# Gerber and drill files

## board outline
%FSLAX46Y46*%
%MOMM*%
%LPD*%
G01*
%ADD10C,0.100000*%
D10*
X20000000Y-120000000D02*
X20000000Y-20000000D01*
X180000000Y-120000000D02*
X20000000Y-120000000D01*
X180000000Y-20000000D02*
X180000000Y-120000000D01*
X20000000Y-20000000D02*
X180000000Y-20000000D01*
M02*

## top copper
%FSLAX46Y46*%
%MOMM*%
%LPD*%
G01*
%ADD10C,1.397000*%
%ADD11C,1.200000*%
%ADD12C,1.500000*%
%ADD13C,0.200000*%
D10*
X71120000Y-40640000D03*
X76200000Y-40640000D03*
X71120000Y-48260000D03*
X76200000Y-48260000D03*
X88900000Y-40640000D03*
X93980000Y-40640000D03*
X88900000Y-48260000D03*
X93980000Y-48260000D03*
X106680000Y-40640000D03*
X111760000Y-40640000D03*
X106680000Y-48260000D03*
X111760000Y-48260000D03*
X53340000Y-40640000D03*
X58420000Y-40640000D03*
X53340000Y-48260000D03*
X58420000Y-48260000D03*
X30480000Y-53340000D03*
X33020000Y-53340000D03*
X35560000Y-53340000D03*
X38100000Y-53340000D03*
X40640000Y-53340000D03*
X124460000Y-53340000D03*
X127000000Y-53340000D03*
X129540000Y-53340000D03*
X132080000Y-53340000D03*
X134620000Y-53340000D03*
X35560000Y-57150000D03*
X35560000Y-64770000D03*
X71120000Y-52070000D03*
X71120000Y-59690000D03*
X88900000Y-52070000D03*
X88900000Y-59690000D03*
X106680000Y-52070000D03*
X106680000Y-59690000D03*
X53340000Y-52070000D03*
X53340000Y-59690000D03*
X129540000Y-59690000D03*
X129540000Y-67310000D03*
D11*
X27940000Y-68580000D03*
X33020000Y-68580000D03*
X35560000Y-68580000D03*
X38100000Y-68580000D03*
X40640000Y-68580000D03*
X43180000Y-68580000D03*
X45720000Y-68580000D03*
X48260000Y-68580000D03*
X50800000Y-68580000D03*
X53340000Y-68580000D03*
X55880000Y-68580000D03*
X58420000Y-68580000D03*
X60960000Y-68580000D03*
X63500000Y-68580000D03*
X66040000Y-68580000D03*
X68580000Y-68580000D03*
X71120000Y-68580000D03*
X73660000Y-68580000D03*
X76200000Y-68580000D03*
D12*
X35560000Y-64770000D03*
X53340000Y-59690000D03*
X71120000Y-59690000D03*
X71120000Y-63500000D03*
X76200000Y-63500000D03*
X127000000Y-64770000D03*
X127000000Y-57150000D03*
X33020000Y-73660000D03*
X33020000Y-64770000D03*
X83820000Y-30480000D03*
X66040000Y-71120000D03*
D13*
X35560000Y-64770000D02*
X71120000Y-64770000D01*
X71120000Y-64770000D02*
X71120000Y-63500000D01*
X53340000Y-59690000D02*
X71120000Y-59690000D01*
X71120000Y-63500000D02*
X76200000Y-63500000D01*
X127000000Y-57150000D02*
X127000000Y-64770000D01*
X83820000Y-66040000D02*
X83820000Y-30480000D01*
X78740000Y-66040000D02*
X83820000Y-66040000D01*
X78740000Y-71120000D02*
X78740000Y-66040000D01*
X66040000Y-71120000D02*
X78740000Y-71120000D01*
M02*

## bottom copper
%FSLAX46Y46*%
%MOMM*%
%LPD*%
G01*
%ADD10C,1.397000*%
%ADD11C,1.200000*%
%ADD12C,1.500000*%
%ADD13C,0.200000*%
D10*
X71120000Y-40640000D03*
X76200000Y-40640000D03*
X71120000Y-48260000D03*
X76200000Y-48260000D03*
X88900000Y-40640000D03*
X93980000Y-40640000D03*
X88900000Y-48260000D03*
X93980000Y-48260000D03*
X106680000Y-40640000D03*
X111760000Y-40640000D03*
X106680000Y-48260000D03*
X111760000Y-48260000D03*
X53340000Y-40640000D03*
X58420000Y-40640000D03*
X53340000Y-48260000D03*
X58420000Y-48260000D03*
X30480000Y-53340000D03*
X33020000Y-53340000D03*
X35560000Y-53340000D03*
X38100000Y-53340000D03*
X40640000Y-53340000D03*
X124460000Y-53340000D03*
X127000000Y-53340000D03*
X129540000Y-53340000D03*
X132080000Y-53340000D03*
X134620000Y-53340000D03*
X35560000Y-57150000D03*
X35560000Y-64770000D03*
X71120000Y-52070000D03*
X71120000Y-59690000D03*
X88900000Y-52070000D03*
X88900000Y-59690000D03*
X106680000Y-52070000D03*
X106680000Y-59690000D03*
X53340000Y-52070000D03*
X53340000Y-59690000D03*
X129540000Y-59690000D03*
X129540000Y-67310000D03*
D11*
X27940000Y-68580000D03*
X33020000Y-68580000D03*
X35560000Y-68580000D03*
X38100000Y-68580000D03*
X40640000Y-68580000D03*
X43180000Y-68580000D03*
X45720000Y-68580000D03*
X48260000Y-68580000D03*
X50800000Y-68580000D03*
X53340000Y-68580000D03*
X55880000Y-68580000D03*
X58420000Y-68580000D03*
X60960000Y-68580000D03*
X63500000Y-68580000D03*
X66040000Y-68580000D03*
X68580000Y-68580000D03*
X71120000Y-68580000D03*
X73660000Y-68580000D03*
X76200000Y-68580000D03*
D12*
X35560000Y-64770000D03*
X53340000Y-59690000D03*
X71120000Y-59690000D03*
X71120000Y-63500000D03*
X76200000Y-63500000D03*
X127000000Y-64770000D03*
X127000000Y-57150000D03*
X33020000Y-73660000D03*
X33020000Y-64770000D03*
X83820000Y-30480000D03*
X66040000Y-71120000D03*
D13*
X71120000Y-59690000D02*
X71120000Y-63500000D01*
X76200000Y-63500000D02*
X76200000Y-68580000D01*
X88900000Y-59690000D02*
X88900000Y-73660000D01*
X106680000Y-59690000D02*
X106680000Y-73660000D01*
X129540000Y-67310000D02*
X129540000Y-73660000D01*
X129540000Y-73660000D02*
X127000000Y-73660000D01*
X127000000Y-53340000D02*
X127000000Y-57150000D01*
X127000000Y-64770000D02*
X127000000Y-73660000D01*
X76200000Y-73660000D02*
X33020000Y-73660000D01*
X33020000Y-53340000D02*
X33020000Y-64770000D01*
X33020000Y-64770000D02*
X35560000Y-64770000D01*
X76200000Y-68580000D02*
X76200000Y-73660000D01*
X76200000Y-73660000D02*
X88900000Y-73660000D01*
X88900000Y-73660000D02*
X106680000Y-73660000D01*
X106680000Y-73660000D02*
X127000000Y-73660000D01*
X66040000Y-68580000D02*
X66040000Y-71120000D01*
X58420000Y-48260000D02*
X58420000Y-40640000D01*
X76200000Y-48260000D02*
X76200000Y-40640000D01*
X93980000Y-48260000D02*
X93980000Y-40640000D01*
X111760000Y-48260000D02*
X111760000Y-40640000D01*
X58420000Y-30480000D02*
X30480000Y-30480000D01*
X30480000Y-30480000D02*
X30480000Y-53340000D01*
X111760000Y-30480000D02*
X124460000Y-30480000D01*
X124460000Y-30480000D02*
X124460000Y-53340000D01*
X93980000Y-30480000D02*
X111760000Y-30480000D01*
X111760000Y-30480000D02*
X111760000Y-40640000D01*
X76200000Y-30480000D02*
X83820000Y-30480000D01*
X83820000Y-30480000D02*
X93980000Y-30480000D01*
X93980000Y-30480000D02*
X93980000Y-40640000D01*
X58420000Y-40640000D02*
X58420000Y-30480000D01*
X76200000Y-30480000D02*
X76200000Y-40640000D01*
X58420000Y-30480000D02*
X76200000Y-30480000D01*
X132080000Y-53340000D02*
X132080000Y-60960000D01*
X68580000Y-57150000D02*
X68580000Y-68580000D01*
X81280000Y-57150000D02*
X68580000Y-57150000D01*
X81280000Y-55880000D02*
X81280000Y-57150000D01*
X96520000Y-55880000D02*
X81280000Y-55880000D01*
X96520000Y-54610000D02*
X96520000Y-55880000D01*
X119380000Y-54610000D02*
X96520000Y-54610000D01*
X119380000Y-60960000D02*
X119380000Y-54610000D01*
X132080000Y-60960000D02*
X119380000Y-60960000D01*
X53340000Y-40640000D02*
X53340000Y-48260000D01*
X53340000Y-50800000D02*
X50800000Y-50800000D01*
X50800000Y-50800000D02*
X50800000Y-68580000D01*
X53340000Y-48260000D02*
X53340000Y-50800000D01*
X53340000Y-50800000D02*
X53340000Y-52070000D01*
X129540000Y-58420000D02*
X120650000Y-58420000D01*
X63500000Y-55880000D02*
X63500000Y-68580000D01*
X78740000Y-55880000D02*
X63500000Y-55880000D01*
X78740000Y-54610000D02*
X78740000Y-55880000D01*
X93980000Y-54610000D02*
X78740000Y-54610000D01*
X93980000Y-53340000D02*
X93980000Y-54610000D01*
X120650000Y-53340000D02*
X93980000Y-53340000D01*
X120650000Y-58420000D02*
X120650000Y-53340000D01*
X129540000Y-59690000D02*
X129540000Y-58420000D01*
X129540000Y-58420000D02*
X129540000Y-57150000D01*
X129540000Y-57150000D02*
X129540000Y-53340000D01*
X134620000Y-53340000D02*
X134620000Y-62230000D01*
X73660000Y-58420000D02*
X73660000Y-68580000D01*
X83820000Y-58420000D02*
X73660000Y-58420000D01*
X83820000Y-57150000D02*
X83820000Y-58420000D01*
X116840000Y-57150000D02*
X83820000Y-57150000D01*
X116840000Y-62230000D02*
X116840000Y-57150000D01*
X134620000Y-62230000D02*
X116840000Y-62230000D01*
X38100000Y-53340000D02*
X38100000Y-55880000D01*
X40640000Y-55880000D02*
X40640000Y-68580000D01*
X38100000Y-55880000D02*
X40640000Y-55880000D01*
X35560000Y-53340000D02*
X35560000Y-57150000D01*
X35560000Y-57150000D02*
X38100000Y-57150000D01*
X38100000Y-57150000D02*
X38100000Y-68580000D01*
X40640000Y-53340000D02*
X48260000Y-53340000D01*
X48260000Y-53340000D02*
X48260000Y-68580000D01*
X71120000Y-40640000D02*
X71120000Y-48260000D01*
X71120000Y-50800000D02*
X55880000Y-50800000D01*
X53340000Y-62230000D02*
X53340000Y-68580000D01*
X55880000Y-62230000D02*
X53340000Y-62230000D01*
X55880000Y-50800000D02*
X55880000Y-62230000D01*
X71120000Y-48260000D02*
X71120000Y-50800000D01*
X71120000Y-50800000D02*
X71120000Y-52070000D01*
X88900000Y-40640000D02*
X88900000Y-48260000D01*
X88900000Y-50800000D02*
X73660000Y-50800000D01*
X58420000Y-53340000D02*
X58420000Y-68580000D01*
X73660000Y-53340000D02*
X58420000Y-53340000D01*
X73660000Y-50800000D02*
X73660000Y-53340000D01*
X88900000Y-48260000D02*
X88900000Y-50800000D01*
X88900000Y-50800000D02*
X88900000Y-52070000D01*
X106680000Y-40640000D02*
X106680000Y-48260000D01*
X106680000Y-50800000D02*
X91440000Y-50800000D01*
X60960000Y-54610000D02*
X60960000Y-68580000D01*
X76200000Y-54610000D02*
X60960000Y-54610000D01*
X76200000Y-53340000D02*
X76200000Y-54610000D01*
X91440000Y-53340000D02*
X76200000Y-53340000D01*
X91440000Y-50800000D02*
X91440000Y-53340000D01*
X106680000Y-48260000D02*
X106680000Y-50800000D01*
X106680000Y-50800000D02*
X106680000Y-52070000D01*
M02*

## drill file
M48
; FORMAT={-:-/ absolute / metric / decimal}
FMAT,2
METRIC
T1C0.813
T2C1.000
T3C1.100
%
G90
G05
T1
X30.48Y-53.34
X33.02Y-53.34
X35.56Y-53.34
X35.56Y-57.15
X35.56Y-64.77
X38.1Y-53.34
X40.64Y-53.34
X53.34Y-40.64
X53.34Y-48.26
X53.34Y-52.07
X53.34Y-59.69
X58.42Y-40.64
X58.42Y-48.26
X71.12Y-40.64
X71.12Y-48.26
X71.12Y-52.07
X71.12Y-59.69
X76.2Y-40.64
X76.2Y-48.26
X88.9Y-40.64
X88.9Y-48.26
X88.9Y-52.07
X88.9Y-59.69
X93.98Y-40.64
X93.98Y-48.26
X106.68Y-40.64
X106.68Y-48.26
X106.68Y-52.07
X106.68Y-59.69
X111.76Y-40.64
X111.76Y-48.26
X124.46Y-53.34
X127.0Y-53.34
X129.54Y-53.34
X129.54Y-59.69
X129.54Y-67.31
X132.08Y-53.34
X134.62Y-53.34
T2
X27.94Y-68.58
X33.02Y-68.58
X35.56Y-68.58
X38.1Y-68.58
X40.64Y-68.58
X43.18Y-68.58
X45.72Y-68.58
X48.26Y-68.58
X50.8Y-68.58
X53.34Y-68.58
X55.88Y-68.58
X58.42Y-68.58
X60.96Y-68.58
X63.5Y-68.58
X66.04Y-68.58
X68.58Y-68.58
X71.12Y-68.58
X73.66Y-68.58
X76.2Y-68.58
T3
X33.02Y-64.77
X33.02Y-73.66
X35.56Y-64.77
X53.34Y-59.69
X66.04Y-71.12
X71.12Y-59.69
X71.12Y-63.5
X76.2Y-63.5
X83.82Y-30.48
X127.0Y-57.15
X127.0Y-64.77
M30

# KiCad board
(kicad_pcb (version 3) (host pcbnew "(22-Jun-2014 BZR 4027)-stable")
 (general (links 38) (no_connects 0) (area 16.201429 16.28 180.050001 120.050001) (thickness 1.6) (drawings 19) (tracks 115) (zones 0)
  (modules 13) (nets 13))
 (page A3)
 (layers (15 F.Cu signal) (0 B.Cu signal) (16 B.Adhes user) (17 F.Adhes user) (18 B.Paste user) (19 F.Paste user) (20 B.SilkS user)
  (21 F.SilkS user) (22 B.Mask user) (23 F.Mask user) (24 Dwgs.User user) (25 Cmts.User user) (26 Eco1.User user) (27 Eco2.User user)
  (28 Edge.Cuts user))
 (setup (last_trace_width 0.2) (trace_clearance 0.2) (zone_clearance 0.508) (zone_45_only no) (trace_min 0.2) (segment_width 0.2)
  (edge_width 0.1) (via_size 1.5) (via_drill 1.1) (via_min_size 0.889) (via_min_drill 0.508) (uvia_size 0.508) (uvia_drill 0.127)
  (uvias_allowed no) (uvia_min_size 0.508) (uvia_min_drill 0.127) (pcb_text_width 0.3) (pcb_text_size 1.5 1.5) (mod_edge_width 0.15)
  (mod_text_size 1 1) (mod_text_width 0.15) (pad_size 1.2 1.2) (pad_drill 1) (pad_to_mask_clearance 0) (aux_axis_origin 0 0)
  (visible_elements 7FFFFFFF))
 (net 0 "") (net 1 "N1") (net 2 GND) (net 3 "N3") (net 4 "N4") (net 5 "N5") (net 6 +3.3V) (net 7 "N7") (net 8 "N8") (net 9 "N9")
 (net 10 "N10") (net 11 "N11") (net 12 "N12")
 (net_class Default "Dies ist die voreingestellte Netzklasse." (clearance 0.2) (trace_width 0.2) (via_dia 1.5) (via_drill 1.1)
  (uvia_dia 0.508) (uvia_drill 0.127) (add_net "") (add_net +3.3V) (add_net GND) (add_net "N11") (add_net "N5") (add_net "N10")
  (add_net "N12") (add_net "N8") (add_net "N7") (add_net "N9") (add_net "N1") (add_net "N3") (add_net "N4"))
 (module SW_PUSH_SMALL (layer F.Cu) (at 73.66 44.45 90)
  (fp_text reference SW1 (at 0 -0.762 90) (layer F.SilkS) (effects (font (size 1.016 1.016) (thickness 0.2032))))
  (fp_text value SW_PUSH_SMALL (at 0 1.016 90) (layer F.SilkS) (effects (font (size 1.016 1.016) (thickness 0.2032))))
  (pad 1 thru_hole circle (at 3.81 -2.54 90) (size 1.397 1.397) (drill 0.8128) (layers *.Cu *.Mask F.SilkS) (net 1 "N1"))
  (pad 2 thru_hole circle (at 3.81 2.54 90) (size 1.397 1.397) (drill 0.8128) (layers *.Cu *.Mask F.SilkS) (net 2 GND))
  (pad 1 thru_hole circle (at -3.81 -2.54 90) (size 1.397 1.397) (drill 0.8128) (layers *.Cu *.Mask F.SilkS) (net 1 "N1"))
  (pad 2 thru_hole circle (at -3.81 2.54 90) (size 1.397 1.397) (drill 0.8128) (layers *.Cu *.Mask F.SilkS) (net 2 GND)))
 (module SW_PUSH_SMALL (layer F.Cu) (at 91.44 44.45 90)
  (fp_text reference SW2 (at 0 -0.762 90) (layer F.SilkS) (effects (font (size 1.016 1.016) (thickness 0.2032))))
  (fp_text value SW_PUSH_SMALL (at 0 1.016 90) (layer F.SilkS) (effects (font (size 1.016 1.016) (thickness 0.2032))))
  (pad 1 thru_hole circle (at 3.81 -2.54 90) (size 1.397 1.397) (drill 0.8128) (layers *.Cu *.Mask F.SilkS) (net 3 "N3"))
  (pad 2 thru_hole circle (at 3.81 2.54 90) (size 1.397 1.397) (drill 0.8128) (layers *.Cu *.Mask F.SilkS) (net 2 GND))
  (pad 1 thru_hole circle (at -3.81 -2.54 90) (size 1.397 1.397) (drill 0.8128) (layers *.Cu *.Mask F.SilkS) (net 3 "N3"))
  (pad 2 thru_hole circle (at -3.81 2.54 90) (size 1.397 1.397) (drill 0.8128) (layers *.Cu *.Mask F.SilkS) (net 2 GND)))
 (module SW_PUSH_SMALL (layer F.Cu) (at 109.22 44.45 90)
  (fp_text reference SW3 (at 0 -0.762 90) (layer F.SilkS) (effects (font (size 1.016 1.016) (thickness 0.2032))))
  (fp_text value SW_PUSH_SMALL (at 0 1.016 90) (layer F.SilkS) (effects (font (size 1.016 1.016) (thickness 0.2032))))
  (pad 1 thru_hole circle (at 3.81 -2.54 90) (size 1.397 1.397) (drill 0.8128) (layers *.Cu *.Mask F.SilkS) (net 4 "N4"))
  (pad 2 thru_hole circle (at 3.81 2.54 90) (size 1.397 1.397) (drill 0.8128) (layers *.Cu *.Mask F.SilkS) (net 2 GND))
  (pad 1 thru_hole circle (at -3.81 -2.54 90) (size 1.397 1.397) (drill 0.8128) (layers *.Cu *.Mask F.SilkS) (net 4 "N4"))
  (pad 2 thru_hole circle (at -3.81 2.54 90) (size 1.397 1.397) (drill 0.8128) (layers *.Cu *.Mask F.SilkS) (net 2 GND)))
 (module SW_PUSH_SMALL (layer F.Cu) (at 55.88 44.45 90)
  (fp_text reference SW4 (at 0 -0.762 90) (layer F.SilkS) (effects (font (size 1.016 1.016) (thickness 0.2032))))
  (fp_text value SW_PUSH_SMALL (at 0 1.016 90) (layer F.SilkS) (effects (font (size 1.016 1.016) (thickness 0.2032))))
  (pad 1 thru_hole circle (at 3.81 -2.54 90) (size 1.397 1.397) (drill 0.8128) (layers *.Cu *.Mask F.SilkS) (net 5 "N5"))
  (pad 2 thru_hole circle (at 3.81 2.54 90) (size 1.397 1.397) (drill 0.8128) (layers *.Cu *.Mask F.SilkS) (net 2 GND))
  (pad 1 thru_hole circle (at -3.81 -2.54 90) (size 1.397 1.397) (drill 0.8128) (layers *.Cu *.Mask F.SilkS) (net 5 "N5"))
  (pad 2 thru_hole circle (at -3.81 2.54 90) (size 1.397 1.397) (drill 0.8128) (layers *.Cu *.Mask F.SilkS) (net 2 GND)))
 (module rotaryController (layer F.Cu) (at 35.56 46.99)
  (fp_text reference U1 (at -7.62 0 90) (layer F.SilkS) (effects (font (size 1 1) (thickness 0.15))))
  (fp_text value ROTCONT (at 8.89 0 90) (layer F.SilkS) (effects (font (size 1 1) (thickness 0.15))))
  (pad 1 thru_hole circle (at -5.08 6.35) (size 1.397 1.397) (drill 0.8128) (layers *.Cu *.Mask F.SilkS) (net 2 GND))
  (pad 2 thru_hole circle (at -2.54 6.35) (size 1.397 1.397) (drill 0.8128) (layers *.Cu *.Mask F.SilkS) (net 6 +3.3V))
  (pad 3 thru_hole circle (at 0 6.35) (size 1.397 1.397) (drill 0.8128) (layers *.Cu *.Mask F.SilkS) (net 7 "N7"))
  (pad 4 thru_hole circle (at 2.54 6.35) (size 1.397 1.397) (drill 0.8128) (layers *.Cu *.Mask F.SilkS) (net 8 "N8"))
  (pad 5 thru_hole circle (at 5.08 6.35) (size 1.397 1.397) (drill 0.8128) (layers *.Cu *.Mask F.SilkS) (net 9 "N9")))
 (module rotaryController (layer F.Cu) (at 129.54 46.99)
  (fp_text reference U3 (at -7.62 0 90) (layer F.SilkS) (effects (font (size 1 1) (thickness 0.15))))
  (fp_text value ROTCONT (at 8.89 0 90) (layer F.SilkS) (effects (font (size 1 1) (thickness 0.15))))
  (pad 1 thru_hole circle (at -5.08 6.35) (size 1.397 1.397) (drill 0.8128) (layers *.Cu *.Mask F.SilkS) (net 2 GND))
  (pad 2 thru_hole circle (at -2.54 6.35) (size 1.397 1.397) (drill 0.8128) (layers *.Cu *.Mask F.SilkS) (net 6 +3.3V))
  (pad 3 thru_hole circle (at 0 6.35) (size 1.397 1.397) (drill 0.8128) (layers *.Cu *.Mask F.SilkS) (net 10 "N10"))
  (pad 4 thru_hole circle (at 2.54 6.35) (size 1.397 1.397) (drill 0.8128) (layers *.Cu *.Mask F.SilkS) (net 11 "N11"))
  (pad 5 thru_hole circle (at 5.08 6.35) (size 1.397 1.397) (drill 0.8128) (layers *.Cu *.Mask F.SilkS) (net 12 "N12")))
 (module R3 (layer F.Cu) (at 35.56 60.96 270) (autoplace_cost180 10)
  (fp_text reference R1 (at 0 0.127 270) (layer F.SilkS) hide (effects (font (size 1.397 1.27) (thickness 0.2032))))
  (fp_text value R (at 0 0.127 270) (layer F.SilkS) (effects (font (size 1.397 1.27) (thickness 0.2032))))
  (pad 1 thru_hole circle (at -3.81 0 270) (size 1.397 1.397) (drill 0.8128) (layers *.Cu *.Mask F.SilkS) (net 7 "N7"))
  (pad 2 thru_hole circle (at 3.81 0 270) (size 1.397 1.397) (drill 0.8128) (layers *.Cu *.Mask F.SilkS) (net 6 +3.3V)))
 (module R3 (layer F.Cu) (at 71.12 55.88 270) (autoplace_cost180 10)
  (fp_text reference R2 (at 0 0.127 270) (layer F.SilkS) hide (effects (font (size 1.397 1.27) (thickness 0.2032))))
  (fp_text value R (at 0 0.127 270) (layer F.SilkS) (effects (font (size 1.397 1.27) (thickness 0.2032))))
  (pad 1 thru_hole circle (at -3.81 0 270) (size 1.397 1.397) (drill 0.8128) (layers *.Cu *.Mask F.SilkS) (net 1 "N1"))
  (pad 2 thru_hole circle (at 3.81 0 270) (size 1.397 1.397) (drill 0.8128) (layers *.Cu *.Mask F.SilkS) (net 6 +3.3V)))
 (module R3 (layer F.Cu) (at 88.9 55.88 270) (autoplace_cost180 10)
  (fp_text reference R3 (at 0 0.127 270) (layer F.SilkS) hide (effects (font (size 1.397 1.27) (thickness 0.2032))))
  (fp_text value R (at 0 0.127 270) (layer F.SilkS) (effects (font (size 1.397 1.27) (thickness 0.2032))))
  (pad 1 thru_hole circle (at -3.81 0 270) (size 1.397 1.397) (drill 0.8128) (layers *.Cu *.Mask F.SilkS) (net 3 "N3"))
  (pad 2 thru_hole circle (at 3.81 0 270) (size 1.397 1.397) (drill 0.8128) (layers *.Cu *.Mask F.SilkS) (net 6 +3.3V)))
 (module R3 (layer F.Cu) (at 106.68 55.88 270) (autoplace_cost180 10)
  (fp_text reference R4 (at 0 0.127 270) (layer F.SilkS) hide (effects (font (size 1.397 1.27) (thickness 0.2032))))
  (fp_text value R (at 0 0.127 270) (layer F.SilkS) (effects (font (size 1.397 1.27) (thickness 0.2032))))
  (pad 1 thru_hole circle (at -3.81 0 270) (size 1.397 1.397) (drill 0.8128) (layers *.Cu *.Mask F.SilkS) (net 4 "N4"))
  (pad 2 thru_hole circle (at 3.81 0 270) (size 1.397 1.397) (drill 0.8128) (layers *.Cu *.Mask F.SilkS) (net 6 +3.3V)))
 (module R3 (layer F.Cu) (at 53.34 55.88 270) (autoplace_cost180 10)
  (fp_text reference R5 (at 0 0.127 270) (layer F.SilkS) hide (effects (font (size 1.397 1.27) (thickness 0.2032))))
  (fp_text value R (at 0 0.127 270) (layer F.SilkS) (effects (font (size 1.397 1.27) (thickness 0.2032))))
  (pad 1 thru_hole circle (at -3.81 0 270) (size 1.397 1.397) (drill 0.8128) (layers *.Cu *.Mask F.SilkS) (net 5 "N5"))
  (pad 2 thru_hole circle (at 3.81 0 270) (size 1.397 1.397) (drill 0.8128) (layers *.Cu *.Mask F.SilkS) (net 6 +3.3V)))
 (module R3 (layer F.Cu) (at 129.54 63.5 270) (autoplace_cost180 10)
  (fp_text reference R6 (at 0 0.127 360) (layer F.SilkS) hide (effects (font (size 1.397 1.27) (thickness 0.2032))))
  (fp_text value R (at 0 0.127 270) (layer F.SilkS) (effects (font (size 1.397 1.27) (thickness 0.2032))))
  (pad 1 thru_hole circle (at -3.81 0 270) (size 1.397 1.397) (drill 0.8128) (layers *.Cu *.Mask F.SilkS) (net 10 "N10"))
  (pad 2 thru_hole circle (at 3.81 0 270) (size 1.397 1.397) (drill 0.8128) (layers *.Cu *.Mask F.SilkS) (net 6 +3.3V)))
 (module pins (layer B.Cu) (at 52.07 68.58)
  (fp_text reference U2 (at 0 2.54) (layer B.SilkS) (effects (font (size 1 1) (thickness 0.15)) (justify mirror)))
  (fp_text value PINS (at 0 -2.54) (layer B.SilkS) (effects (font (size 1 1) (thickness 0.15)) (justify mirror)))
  (pad 1 thru_hole circle (at -24.13 0) (size 1.2 1.2) (drill 1) (layers *.Cu *.Mask B.SilkS))
  (pad 3 thru_hole circle (at -19.05 0) (size 1.2 1.2) (drill 1) (layers *.Cu *.Mask B.SilkS))
  (pad 4 thru_hole circle (at -16.51 0) (size 1.2 1.2) (drill 1) (layers *.Cu *.Mask B.SilkS))
  (pad 5 thru_hole circle (at -13.97 0) (size 1.2 1.2) (drill 1) (layers *.Cu *.Mask B.SilkS) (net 7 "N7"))
  (pad 6 thru_hole circle (at -11.43 0) (size 1.2 1.2) (drill 1) (layers *.Cu *.Mask B.SilkS) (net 8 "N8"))
  (pad 7 thru_hole circle (at -8.89 0) (size 1.2 1.2) (drill 1) (layers *.Cu *.Mask B.SilkS))
  (pad 8 thru_hole circle (at -6.35 0) (size 1.2 1.2) (drill 1) (layers *.Cu *.Mask B.SilkS))
  (pad 9 thru_hole circle (at -3.81 0) (size 1.2 1.2) (drill 1) (layers *.Cu *.Mask B.SilkS) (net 9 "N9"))
  (pad 10 thru_hole circle (at -1.27 0) (size 1.2 1.2) (drill 1) (layers *.Cu *.Mask B.SilkS) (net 5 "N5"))
  (pad 11 thru_hole circle (at 1.27 0) (size 1.2 1.2) (drill 1) (layers *.Cu *.Mask B.SilkS) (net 1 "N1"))
  (pad 12 thru_hole circle (at 3.81 0) (size 1.2 1.2) (drill 1) (layers *.Cu *.Mask B.SilkS))
  (pad 13 thru_hole circle (at 6.35 0) (size 1.2 1.2) (drill 1) (layers *.Cu *.Mask B.SilkS) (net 3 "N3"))
  (pad 14 thru_hole circle (at 8.89 0) (size 1.2 1.2) (drill 1) (layers *.Cu *.Mask B.SilkS) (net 4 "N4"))
  (pad 15 thru_hole circle (at 11.43 0) (size 1.2 1.2) (drill 1) (layers *.Cu *.Mask B.SilkS) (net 10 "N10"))
  (pad 16 thru_hole circle (at 13.97 0) (size 1.2 1.2) (drill 1) (layers *.Cu *.Mask B.SilkS) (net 2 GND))
  (pad 17 thru_hole circle (at 16.51 0) (size 1.2 1.2) (drill 1) (layers *.Cu *.Mask B.SilkS) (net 11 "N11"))
  (pad 18 thru_hole circle (at 19.05 0) (size 1.2 1.2) (drill 1) (layers *.Cu *.Mask B.SilkS))
  (pad 19 thru_hole circle (at 21.59 0) (size 1.2 1.2) (drill 1) (layers *.Cu *.Mask B.SilkS) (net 12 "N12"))
  (pad 20 thru_hole circle (at 24.13 0) (size 1.2 1.2) (drill 1) (layers *.Cu *.Mask B.SilkS) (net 6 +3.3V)))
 (gr_line (start 20 120) (end 20 20) (angle 90) (layer Edge.Cuts) (width 0.1))
 (gr_line (start 180 120) (end 20 120) (angle 90) (layer Edge.Cuts) (width 0.1))
 (gr_line (start 180 20) (end 180 120) (angle 90) (layer Edge.Cuts) (width 0.1))
 (gr_line (start 20 20) (end 180 20) (angle 90) (layer Edge.Cuts) (width 0.1))
 (via (at 35.56 64.77) (size 1.5) (layers F.Cu B.Cu) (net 6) (status C00000))
 (segment (start 35.56 64.77) (end 71.12 64.77) (width 0.2) (layer F.Cu) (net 6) (status 400000))
 (segment (start 71.12 64.77) (end 71.12 63.5) (width 0.2) (layer F.Cu) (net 6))
 (via (at 53.34 59.69) (size 1.5) (layers F.Cu B.Cu) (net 6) (status C00000))
 (segment (start 53.34 59.69) (end 71.12 59.69) (width 0.2) (layer F.Cu) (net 6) (status C00000))
 (via (at 71.12 59.69) (size 1.5) (layers F.Cu B.Cu) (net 6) (status C00000))
 (segment (start 71.12 59.69) (end 71.12 63.5) (width 0.2) (layer B.Cu) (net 6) (status 400000))
 (via (at 71.12 63.5) (size 1.5) (layers F.Cu B.Cu) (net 6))
 (segment (start 71.12 63.5) (end 76.2 63.5) (width 0.2) (layer F.Cu) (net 6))
 (segment (start 76.2 63.5) (end 76.2 68.58) (width 0.2) (layer B.Cu) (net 6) (status 800000))
 (via (at 76.2 63.5) (size 1.5) (layers F.Cu B.Cu) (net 6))
 (segment (start 88.9 59.69) (end 88.9 73.66) (width 0.2) (layer B.Cu) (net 6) (status 400000))
 (segment (start 106.68 59.69) (end 106.68 73.66) (width 0.2) (layer B.Cu) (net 6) (status 400000))
 (segment (start 129.54 67.31) (end 129.54 73.66) (width 0.2) (layer B.Cu) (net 6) (status 400000))
 (segment (start 129.54 73.66) (end 127 73.66) (width 0.2) (layer B.Cu) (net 6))
 (segment (start 127 53.34) (end 127 57.15) (width 0.2) (layer B.Cu) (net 6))
 (segment (start 127 64.77) (end 127 73.66) (width 0.2) (layer B.Cu) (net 6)) (via (at 127 64.77) (size 1.5) (layers F.Cu B.Cu) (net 6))
 (segment (start 127 57.15) (end 127 64.77) (width 0.2) (layer F.Cu) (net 6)) (via (at 127 57.15) (size 1.5) (layers F.Cu B.Cu) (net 6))
 (segment (start 76.2 73.66) (end 33.02 73.66) (width 0.2) (layer B.Cu) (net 6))
 (via (at 33.02 73.66) (size 1.5) (layers F.Cu B.Cu) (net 6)) (via (at 33.02 64.77) (size 1.5) (layers F.Cu B.Cu) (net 6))
 (segment (start 33.02 53.34) (end 33.02 64.77) (width 0.2) (layer B.Cu) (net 6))
 (segment (start 33.02 64.77) (end 35.56 64.77) (width 0.2) (layer B.Cu) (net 6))
 (segment (start 76.2 68.58) (end 76.2 73.66) (width 0.2) (layer B.Cu) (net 6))
 (segment (start 76.2 73.66) (end 88.9 73.66) (width 0.2) (layer B.Cu) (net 6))
 (segment (start 88.9 73.66) (end 106.68 73.66) (width 0.2) (layer B.Cu) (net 6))
 (segment (start 106.68 73.66) (end 127 73.66) (width 0.2) (layer B.Cu) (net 6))
 (segment (start 66.04 68.58) (end 66.04 71.12) (width 0.2) (layer B.Cu) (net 2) (status 400000))
 (via (at 83.82 30.48) (size 1.5) (layers F.Cu B.Cu) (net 2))
 (segment (start 83.82 66.04) (end 83.82 30.48) (width 0.2) (layer F.Cu) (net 2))
 (segment (start 78.74 66.04) (end 83.82 66.04) (width 0.2) (layer F.Cu) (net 2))
 (segment (start 78.74 71.12) (end 78.74 66.04) (width 0.2) (layer F.Cu) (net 2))
 (segment (start 66.04 71.12) (end 78.74 71.12) (width 0.2) (layer F.Cu) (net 2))
 (via (at 66.04 71.12) (size 1.5) (layers F.Cu B.Cu) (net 2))
 (segment (start 58.42 48.26) (end 58.42 40.64) (width 0.2) (layer B.Cu) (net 2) (status C00000))
 (segment (start 76.2 48.26) (end 76.2 40.64) (width 0.2) (layer B.Cu) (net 2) (status C00000))
 (segment (start 93.98 48.26) (end 93.98 40.64) (width 0.2) (layer B.Cu) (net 2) (status C00000))
 (segment (start 111.76 48.26) (end 111.76 40.64) (width 0.2) (layer B.Cu) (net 2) (status C00000))
 (segment (start 58.42 30.48) (end 30.48 30.48) (width 0.2) (layer B.Cu) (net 2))
 (segment (start 30.48 30.48) (end 30.48 53.34) (width 0.2) (layer B.Cu) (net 2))
 (segment (start 111.76 30.48) (end 124.46 30.48) (width 0.2) (layer B.Cu) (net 2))
 (segment (start 124.46 30.48) (end 124.46 53.34) (width 0.2) (layer B.Cu) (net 2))
 (segment (start 93.98 30.48) (end 111.76 30.48) (width 0.2) (layer B.Cu) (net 2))
 (segment (start 111.76 30.48) (end 111.76 40.64) (width 0.2) (layer B.Cu) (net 2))
 (segment (start 76.2 30.48) (end 83.82 30.48) (width 0.2) (layer B.Cu) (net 2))
 (segment (start 83.82 30.48) (end 93.98 30.48) (width 0.2) (layer B.Cu) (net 2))
 (segment (start 93.98 30.48) (end 93.98 40.64) (width 0.2) (layer B.Cu) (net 2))
 (segment (start 58.42 40.64) (end 58.42 30.48) (width 0.2) (layer B.Cu) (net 2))
 (segment (start 76.2 30.48) (end 76.2 40.64) (width 0.2) (layer B.Cu) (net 2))
 (segment (start 58.42 30.48) (end 76.2 30.48) (width 0.2) (layer B.Cu) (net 2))
 (segment (start 132.08 53.34) (end 132.08 60.96) (width 0.2) (layer B.Cu) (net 11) (status 400000))
 (segment (start 68.58 57.15) (end 68.58 68.58) (width 0.2) (layer B.Cu) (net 11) (status 800000))
 (segment (start 81.28 57.15) (end 68.58 57.15) (width 0.2) (layer B.Cu) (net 11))
 (segment (start 81.28 55.88) (end 81.28 57.15) (width 0.2) (layer B.Cu) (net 11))
 (segment (start 96.52 55.88) (end 81.28 55.88) (width 0.2) (layer B.Cu) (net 11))
 (segment (start 96.52 54.61) (end 96.52 55.88) (width 0.2) (layer B.Cu) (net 11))
 (segment (start 119.38 54.61) (end 96.52 54.61) (width 0.2) (layer B.Cu) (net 11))
 (segment (start 119.38 60.96) (end 119.38 54.61) (width 0.2) (layer B.Cu) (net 11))
 (segment (start 132.08 60.96) (end 119.38 60.96) (width 0.2) (layer B.Cu) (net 11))
 (segment (start 53.34 40.64) (end 53.34 48.26) (width 0.2) (layer B.Cu) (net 5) (status C00000))
 (segment (start 53.34 50.8) (end 50.8 50.8) (width 0.2) (layer B.Cu) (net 5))
 (segment (start 50.8 50.8) (end 50.8 68.58) (width 0.2) (layer B.Cu) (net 5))
 (segment (start 53.34 48.26) (end 53.34 50.8) (width 0.2) (layer B.Cu) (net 5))
 (segment (start 53.34 50.8) (end 53.34 52.07) (width 0.2) (layer B.Cu) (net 5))
 (segment (start 129.54 58.42) (end 120.65 58.42) (width 0.2) (layer B.Cu) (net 10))
 (segment (start 63.5 55.88) (end 63.5 68.58) (width 0.2) (layer B.Cu) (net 10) (status 800000))
 (segment (start 78.74 55.88) (end 63.5 55.88) (width 0.2) (layer B.Cu) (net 10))
 (segment (start 78.74 54.61) (end 78.74 55.88) (width 0.2) (layer B.Cu) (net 10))
 (segment (start 93.98 54.61) (end 78.74 54.61) (width 0.2) (layer B.Cu) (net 10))
 (segment (start 93.98 53.34) (end 93.98 54.61) (width 0.2) (layer B.Cu) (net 10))
 (segment (start 120.65 53.34) (end 93.98 53.34) (width 0.2) (layer B.Cu) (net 10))
 (segment (start 120.65 58.42) (end 120.65 53.34) (width 0.2) (layer B.Cu) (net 10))
 (segment (start 129.54 59.69) (end 129.54 58.42) (width 0.2) (layer B.Cu) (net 10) (status 400000))
 (segment (start 129.54 58.42) (end 129.54 57.15) (width 0.2) (layer B.Cu) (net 10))
 (segment (start 129.54 57.15) (end 129.54 53.34) (width 0.2) (layer B.Cu) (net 10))
 (segment (start 134.62 53.34) (end 134.62 62.23) (width 0.2) (layer B.Cu) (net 12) (status 400000))
 (segment (start 73.66 58.42) (end 73.66 68.58) (width 0.2) (layer B.Cu) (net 12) (status 800000))
 (segment (start 83.82 58.42) (end 73.66 58.42) (width 0.2) (layer B.Cu) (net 12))
 (segment (start 83.82 57.15) (end 83.82 58.42) (width 0.2) (layer B.Cu) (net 12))
 (segment (start 116.84 57.15) (end 83.82 57.15) (width 0.2) (layer B.Cu) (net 12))
 (segment (start 116.84 62.23) (end 116.84 57.15) (width 0.2) (layer B.Cu) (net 12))
 (segment (start 134.62 62.23) (end 116.84 62.23) (width 0.2) (layer B.Cu) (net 12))
 (segment (start 38.1 53.34) (end 38.1 55.88) (width 0.2) (layer B.Cu) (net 8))
 (segment (start 40.64 55.88) (end 40.64 68.58) (width 0.2) (layer B.Cu) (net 8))
 (segment (start 38.1 55.88) (end 40.64 55.88) (width 0.2) (layer B.Cu) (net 8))
 (segment (start 35.56 53.34) (end 35.56 57.15) (width 0.2) (layer B.Cu) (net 7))
 (segment (start 35.56 57.15) (end 38.1 57.15) (width 0.2) (layer B.Cu) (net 7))
 (segment (start 38.1 57.15) (end 38.1 68.58) (width 0.2) (layer B.Cu) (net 7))
 (segment (start 40.64 53.34) (end 48.26 53.34) (width 0.2) (layer B.Cu) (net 9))
 (segment (start 48.26 53.34) (end 48.26 68.58) (width 0.2) (layer B.Cu) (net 9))
 (segment (start 71.12 40.64) (end 71.12 48.26) (width 0.2) (layer B.Cu) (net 1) (status C00000))
 (segment (start 71.12 50.8) (end 55.88 50.8) (width 0.2) (layer B.Cu) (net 1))
 (segment (start 53.34 62.23) (end 53.34 68.58) (width 0.2) (layer B.Cu) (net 1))
 (segment (start 55.88 62.23) (end 53.34 62.23) (width 0.2) (layer B.Cu) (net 1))
 (segment (start 55.88 50.8) (end 55.88 62.23) (width 0.2) (layer B.Cu) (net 1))
 (segment (start 71.12 48.26) (end 71.12 50.8) (width 0.2) (layer B.Cu) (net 1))
 (segment (start 71.12 50.8) (end 71.12 52.07) (width 0.2) (layer B.Cu) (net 1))
 (segment (start 88.9 40.64) (end 88.9 48.26) (width 0.2) (layer B.Cu) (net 3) (status C00000))
 (segment (start 88.9 50.8) (end 73.66 50.8) (width 0.2) (layer B.Cu) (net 3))
 (segment (start 58.42 53.34) (end 58.42 68.58) (width 0.2) (layer B.Cu) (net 3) (status 800000))
 (segment (start 73.66 53.34) (end 58.42 53.34) (width 0.2) (layer B.Cu) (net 3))
 (segment (start 73.66 50.8) (end 73.66 53.34) (width 0.2) (layer B.Cu) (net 3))
 (segment (start 88.9 48.26) (end 88.9 50.8) (width 0.2) (layer B.Cu) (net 3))
 (segment (start 88.9 50.8) (end 88.9 52.07) (width 0.2) (layer B.Cu) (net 3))
 (segment (start 106.68 40.64) (end 106.68 48.26) (width 0.2) (layer B.Cu) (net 4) (status C00000))
 (segment (start 106.68 50.8) (end 91.44 50.8) (width 0.2) (layer B.Cu) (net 4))
 (segment (start 60.96 54.61) (end 60.96 68.58) (width 0.2) (layer B.Cu) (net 4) (status 800000))
 (segment (start 76.2 54.61) (end 60.96 54.61) (width 0.2) (layer B.Cu) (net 4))
 (segment (start 76.2 53.34) (end 76.2 54.61) (width 0.2) (layer B.Cu) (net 4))
 (segment (start 91.44 53.34) (end 76.2 53.34) (width 0.2) (layer B.Cu) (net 4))
 (segment (start 91.44 50.8) (end 91.44 53.34) (width 0.2) (layer B.Cu) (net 4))
 (segment (start 106.68 48.26) (end 106.68 50.8) (width 0.2) (layer B.Cu) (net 4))
 (segment (start 106.68 50.8) (end 106.68 52.07) (width 0.2) (layer B.Cu) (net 4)))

